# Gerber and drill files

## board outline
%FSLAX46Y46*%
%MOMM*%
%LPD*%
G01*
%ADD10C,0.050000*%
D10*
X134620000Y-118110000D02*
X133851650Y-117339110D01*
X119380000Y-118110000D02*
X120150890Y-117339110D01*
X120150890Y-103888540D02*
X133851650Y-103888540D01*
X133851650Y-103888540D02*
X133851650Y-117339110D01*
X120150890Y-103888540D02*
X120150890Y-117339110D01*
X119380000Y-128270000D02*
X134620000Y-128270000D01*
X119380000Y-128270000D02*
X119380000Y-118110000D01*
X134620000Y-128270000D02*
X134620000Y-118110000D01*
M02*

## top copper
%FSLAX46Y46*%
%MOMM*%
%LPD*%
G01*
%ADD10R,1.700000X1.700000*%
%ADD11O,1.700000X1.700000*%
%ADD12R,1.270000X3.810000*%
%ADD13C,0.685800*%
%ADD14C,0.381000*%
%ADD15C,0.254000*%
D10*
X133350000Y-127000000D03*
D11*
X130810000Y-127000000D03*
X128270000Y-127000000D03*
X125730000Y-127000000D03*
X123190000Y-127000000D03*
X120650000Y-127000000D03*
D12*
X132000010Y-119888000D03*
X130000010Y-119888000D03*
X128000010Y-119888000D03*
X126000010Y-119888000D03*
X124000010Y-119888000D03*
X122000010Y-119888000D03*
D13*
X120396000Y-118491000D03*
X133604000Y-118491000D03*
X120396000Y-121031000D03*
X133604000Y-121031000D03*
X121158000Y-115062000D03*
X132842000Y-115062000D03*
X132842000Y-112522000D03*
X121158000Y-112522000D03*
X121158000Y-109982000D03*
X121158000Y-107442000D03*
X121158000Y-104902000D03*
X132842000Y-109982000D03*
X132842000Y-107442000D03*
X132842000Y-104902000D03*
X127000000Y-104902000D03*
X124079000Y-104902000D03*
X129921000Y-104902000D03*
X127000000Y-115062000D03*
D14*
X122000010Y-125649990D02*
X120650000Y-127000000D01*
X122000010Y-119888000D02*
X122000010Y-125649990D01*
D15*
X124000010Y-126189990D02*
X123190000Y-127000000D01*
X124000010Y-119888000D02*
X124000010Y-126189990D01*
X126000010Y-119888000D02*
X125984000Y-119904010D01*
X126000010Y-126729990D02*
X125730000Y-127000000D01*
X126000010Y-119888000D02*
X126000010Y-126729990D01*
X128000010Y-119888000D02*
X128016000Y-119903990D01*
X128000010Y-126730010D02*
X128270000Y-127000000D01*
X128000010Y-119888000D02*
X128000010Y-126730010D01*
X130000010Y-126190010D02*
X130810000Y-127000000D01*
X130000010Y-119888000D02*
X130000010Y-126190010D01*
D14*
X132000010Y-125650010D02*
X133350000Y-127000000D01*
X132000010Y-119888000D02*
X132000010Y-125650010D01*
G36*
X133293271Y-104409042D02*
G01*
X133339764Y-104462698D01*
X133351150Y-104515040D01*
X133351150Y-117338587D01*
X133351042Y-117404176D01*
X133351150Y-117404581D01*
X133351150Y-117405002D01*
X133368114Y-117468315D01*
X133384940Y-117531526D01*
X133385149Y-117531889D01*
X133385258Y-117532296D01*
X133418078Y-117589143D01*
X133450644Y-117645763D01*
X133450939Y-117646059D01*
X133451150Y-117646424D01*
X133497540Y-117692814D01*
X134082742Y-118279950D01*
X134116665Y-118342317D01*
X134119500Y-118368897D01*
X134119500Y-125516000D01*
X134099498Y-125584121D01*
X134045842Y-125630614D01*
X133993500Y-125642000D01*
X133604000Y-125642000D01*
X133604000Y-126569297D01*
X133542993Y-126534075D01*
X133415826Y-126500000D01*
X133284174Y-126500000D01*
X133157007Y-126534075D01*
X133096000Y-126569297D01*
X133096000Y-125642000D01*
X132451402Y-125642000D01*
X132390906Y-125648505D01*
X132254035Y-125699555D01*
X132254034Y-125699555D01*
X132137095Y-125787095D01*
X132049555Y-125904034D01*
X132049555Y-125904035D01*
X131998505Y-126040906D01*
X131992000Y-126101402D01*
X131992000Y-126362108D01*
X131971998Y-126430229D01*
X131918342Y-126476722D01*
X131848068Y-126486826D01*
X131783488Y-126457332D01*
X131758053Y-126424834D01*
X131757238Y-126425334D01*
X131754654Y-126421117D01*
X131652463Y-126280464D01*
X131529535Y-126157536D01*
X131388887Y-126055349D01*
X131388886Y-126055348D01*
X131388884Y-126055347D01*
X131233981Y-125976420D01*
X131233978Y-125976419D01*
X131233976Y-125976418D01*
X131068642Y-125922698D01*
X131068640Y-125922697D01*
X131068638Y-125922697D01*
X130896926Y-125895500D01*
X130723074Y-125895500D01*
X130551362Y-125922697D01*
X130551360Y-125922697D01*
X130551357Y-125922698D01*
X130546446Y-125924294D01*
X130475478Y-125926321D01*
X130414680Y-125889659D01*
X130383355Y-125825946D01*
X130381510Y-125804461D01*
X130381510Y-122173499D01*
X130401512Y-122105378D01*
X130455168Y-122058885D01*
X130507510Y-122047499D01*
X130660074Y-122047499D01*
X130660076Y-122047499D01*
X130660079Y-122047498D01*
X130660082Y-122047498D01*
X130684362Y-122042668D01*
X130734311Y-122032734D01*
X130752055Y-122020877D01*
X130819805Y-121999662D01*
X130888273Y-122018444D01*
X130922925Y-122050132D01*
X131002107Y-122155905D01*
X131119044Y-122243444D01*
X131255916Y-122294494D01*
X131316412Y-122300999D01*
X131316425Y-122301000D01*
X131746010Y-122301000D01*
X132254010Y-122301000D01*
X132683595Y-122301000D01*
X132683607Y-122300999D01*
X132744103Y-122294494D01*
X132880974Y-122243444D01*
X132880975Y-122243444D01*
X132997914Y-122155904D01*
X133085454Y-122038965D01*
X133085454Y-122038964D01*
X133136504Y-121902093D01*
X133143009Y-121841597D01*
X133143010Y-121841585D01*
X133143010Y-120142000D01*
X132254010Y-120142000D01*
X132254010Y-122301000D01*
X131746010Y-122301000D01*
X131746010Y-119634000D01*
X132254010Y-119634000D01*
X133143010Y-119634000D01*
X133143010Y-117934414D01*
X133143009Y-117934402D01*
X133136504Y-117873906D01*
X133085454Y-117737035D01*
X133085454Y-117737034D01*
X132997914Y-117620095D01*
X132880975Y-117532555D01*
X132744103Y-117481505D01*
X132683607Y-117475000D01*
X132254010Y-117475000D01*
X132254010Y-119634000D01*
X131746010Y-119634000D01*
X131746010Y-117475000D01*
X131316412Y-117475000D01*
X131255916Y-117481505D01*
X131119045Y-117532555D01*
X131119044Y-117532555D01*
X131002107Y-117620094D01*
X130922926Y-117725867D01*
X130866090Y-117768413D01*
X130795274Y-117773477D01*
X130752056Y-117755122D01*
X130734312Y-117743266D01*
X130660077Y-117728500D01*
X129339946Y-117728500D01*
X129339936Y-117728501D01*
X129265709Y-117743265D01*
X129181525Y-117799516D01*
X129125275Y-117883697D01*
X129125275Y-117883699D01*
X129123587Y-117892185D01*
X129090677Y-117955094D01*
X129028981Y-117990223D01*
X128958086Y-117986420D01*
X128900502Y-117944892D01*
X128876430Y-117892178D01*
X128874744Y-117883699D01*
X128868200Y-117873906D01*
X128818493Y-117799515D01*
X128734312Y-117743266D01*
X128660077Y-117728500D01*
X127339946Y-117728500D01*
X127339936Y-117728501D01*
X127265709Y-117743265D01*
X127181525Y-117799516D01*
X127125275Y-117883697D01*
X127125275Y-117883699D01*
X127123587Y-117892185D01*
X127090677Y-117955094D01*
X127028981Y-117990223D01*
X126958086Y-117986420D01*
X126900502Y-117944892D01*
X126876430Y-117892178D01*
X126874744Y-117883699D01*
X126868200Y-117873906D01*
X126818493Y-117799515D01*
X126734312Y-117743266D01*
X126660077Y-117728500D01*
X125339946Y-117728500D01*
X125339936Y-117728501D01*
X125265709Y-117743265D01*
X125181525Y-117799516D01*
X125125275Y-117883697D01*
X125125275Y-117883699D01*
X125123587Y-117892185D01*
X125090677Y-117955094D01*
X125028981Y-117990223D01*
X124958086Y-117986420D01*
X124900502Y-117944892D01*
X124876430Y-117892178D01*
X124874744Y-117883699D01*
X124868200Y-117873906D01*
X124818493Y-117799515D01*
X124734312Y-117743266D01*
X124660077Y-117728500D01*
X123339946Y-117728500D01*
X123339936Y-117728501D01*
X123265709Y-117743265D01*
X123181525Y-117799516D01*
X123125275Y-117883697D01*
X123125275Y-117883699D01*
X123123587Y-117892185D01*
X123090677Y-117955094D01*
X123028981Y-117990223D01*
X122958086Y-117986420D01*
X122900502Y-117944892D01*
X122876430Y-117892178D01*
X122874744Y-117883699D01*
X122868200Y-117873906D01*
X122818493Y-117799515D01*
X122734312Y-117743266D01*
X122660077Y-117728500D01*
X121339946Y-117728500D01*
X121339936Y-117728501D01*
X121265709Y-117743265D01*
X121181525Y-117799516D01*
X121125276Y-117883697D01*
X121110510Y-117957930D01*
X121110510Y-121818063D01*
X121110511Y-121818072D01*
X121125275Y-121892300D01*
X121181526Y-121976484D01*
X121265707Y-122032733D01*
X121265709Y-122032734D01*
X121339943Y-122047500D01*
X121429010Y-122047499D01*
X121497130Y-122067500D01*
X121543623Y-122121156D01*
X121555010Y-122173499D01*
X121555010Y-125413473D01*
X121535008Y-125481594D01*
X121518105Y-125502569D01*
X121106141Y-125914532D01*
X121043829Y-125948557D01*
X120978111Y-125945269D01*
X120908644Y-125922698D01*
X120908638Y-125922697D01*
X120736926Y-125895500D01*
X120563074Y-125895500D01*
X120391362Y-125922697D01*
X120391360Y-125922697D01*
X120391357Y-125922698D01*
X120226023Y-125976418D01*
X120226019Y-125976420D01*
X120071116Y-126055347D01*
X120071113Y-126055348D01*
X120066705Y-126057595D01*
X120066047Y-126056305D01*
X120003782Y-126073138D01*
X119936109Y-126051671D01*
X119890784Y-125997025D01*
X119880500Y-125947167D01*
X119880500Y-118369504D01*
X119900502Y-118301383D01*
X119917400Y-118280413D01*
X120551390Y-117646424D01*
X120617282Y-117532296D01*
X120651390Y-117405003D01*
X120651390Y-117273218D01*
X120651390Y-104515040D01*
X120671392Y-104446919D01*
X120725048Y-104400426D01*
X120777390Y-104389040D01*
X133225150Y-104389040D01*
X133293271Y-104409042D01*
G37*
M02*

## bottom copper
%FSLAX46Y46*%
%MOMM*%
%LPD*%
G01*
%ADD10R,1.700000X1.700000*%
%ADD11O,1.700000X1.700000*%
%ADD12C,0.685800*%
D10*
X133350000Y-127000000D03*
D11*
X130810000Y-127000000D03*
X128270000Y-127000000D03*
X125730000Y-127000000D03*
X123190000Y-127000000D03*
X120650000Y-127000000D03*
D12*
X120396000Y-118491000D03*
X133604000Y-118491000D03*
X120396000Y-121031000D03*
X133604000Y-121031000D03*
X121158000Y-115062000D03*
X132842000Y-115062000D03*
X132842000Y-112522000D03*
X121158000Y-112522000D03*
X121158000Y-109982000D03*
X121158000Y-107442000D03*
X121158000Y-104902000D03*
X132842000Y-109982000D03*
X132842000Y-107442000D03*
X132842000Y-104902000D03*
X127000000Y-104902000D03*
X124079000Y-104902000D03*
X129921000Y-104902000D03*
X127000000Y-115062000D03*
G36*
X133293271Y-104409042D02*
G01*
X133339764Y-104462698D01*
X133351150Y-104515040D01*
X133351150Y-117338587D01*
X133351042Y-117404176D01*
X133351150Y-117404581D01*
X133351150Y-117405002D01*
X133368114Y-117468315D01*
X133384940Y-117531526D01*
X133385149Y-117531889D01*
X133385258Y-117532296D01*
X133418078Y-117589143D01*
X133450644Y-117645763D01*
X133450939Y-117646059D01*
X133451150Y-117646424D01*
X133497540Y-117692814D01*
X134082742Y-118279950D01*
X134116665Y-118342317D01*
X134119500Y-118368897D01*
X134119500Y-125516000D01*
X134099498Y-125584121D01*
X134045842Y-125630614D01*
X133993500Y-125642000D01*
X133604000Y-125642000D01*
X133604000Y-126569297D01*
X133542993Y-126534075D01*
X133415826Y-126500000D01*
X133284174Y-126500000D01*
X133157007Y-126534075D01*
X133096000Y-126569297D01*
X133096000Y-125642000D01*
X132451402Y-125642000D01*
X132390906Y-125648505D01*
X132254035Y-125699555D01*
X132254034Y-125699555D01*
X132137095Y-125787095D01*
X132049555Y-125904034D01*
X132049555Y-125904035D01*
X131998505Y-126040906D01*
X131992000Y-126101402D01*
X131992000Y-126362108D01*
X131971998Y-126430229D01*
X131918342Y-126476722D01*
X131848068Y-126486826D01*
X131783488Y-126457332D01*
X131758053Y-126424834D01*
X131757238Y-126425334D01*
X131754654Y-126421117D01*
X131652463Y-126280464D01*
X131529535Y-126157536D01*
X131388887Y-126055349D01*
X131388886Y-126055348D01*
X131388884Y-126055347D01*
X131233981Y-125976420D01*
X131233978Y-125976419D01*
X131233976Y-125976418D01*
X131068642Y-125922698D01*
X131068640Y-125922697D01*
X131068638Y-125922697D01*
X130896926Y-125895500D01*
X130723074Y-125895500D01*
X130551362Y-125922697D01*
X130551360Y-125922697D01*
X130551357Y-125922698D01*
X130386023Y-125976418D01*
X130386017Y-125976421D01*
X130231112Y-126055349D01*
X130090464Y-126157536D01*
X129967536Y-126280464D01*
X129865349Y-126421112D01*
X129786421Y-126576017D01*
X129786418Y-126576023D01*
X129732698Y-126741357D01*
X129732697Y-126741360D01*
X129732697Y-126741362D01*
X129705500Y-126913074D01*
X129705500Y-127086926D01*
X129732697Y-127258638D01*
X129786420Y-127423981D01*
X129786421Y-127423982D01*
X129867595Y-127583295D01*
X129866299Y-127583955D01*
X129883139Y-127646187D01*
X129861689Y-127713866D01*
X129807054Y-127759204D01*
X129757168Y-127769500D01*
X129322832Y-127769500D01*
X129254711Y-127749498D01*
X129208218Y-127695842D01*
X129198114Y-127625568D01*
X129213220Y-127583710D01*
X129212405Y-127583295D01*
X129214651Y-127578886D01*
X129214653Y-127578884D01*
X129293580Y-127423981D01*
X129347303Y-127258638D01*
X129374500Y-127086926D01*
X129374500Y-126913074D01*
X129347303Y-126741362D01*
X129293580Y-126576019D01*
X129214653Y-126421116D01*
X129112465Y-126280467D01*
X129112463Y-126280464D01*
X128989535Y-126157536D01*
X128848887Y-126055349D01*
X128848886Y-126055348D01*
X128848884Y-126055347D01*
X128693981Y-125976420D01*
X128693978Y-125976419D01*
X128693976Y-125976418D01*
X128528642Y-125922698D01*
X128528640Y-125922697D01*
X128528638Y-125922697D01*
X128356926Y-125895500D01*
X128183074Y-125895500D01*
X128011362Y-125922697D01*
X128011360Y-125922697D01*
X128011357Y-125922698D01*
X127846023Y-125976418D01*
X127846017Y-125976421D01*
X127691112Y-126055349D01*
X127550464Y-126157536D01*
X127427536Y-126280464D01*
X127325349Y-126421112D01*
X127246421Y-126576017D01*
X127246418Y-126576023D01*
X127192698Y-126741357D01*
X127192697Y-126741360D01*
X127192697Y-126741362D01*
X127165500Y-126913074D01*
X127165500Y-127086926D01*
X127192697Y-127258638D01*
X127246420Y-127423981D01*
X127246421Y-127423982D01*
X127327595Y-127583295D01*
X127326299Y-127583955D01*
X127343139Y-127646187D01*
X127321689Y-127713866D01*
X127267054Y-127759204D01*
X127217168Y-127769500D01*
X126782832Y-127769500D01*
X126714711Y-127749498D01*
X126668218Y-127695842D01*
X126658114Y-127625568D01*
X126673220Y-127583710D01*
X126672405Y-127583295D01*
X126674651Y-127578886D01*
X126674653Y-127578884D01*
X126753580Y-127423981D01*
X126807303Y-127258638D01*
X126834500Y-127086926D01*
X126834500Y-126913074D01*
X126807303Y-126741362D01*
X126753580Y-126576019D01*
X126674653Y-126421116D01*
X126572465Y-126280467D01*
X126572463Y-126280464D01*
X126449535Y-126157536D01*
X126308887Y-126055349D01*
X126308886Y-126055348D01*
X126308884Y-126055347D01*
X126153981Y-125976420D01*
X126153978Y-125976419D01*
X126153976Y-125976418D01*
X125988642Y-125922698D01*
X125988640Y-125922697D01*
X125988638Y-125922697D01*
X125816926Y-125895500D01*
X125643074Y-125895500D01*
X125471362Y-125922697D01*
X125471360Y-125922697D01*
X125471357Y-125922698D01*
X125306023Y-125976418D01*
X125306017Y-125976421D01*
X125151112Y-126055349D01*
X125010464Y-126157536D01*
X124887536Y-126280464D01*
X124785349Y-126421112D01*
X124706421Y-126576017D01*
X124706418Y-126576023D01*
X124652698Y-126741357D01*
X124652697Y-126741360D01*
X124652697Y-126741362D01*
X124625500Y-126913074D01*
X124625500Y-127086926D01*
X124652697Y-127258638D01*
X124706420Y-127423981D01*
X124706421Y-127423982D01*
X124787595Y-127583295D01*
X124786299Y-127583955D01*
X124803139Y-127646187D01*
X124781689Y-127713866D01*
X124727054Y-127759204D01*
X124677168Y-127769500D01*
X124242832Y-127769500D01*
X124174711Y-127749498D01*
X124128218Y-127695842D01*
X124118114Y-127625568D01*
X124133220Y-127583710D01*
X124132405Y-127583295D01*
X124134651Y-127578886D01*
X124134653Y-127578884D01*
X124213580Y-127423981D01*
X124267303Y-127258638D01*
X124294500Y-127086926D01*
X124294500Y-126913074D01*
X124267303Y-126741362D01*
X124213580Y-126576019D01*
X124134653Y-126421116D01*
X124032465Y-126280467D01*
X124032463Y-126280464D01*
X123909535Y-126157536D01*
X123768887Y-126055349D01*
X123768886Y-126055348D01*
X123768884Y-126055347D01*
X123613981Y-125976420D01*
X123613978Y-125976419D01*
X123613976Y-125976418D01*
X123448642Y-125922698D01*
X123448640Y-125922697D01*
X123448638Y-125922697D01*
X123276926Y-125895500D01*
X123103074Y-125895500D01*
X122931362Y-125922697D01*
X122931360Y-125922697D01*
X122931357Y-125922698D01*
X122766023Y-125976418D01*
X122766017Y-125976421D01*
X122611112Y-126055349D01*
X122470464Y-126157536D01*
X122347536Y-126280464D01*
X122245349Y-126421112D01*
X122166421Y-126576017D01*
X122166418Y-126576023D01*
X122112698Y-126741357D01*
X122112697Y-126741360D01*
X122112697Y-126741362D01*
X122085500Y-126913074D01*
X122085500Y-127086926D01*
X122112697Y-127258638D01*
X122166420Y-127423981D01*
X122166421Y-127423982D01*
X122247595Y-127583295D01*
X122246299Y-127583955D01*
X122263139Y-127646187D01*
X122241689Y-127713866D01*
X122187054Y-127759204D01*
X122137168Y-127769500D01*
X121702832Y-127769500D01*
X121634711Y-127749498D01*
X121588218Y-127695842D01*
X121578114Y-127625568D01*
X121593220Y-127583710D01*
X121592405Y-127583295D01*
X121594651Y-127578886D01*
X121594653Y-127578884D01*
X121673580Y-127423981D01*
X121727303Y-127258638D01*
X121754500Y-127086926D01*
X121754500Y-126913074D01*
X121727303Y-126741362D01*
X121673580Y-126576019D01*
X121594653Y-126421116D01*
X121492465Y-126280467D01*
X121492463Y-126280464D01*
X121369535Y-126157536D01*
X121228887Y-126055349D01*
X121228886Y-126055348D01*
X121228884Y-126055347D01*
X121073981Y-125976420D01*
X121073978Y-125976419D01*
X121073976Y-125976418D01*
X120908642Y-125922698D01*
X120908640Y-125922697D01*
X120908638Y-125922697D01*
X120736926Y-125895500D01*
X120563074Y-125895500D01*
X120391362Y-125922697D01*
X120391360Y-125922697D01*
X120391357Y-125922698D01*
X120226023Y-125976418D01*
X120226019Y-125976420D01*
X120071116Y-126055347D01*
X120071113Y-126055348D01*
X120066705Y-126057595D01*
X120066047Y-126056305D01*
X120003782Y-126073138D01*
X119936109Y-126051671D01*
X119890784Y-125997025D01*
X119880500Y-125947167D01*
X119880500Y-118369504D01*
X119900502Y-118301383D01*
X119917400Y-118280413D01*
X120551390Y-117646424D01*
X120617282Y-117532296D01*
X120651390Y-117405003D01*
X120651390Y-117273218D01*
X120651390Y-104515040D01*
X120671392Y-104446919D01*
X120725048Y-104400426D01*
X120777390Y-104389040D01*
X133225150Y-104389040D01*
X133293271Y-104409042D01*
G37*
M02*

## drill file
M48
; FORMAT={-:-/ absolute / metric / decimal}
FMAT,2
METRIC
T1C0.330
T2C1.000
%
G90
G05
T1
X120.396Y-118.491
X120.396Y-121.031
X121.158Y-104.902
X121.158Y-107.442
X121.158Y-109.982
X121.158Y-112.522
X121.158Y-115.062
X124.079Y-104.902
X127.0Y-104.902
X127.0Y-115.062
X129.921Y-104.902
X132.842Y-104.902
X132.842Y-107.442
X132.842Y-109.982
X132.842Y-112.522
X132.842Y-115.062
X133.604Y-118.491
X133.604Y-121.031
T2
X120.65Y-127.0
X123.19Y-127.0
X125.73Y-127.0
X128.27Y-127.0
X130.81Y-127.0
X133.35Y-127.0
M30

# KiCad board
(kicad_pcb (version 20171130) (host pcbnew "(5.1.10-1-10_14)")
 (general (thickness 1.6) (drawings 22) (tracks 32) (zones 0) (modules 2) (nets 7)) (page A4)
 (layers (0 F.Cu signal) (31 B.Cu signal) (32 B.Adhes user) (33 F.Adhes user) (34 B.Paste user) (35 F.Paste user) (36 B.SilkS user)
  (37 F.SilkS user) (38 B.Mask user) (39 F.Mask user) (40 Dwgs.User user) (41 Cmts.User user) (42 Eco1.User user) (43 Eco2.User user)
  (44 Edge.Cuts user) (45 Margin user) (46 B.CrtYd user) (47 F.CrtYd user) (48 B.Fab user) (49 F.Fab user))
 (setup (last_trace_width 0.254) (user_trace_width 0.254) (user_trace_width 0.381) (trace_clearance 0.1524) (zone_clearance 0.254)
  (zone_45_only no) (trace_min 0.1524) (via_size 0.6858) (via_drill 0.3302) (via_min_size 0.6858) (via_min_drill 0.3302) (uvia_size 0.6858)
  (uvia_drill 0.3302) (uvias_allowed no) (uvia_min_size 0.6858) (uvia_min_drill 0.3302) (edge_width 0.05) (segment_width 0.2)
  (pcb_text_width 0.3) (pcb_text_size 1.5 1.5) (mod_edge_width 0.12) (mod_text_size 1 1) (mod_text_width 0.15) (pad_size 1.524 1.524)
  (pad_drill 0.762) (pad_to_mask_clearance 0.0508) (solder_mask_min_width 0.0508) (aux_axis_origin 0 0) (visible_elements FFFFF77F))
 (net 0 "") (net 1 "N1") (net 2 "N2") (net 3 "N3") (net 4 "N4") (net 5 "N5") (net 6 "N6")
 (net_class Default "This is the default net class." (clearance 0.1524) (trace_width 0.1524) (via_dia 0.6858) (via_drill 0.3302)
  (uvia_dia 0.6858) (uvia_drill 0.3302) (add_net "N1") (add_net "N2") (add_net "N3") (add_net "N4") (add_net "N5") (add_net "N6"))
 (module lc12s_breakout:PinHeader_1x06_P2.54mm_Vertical (layer F.Cu) (at 133.35 127 270)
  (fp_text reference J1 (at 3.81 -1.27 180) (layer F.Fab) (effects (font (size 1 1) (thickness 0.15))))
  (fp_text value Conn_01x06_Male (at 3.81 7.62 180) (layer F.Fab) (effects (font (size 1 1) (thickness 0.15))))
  (pad 1 thru_hole rect (at 0 0 270) (size 1.7 1.7) (drill 1) (layers *.Cu *.Mask) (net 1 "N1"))
  (pad 2 thru_hole oval (at 0 2.54 270) (size 1.7 1.7) (drill 1) (layers *.Cu *.Mask) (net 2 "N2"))
  (pad 3 thru_hole oval (at 0 5.08 270) (size 1.7 1.7) (drill 1) (layers *.Cu *.Mask) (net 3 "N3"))
  (pad 4 thru_hole oval (at 0 7.62 270) (size 1.7 1.7) (drill 1) (layers *.Cu *.Mask) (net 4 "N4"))
  (pad 5 thru_hole oval (at 0 10.16 270) (size 1.7 1.7) (drill 1) (layers *.Cu *.Mask) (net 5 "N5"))
  (pad 6 thru_hole oval (at 0 12.7 270) (size 1.7 1.7) (drill 1) (layers *.Cu *.Mask) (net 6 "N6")))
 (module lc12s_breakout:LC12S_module (layer F.Cu) (at 122.00001 119.888)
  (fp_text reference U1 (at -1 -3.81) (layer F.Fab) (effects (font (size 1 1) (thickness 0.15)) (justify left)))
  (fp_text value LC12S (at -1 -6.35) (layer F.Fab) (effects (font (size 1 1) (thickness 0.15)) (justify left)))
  (pad 6 smd rect (at 10 0) (size 1.27 3.81) (layers F.Cu F.Paste F.Mask) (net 1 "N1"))
  (pad 5 smd rect (at 8 0) (size 1.27 3.81) (layers F.Cu F.Paste F.Mask) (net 2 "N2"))
  (pad 4 smd rect (at 6 0) (size 1.27 3.81) (layers F.Cu F.Paste F.Mask) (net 3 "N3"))
  (pad 3 smd rect (at 4 0) (size 1.27 3.81) (layers F.Cu F.Paste F.Mask) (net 4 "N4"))
  (pad 2 smd rect (at 2 0) (size 1.27 3.81) (layers F.Cu F.Paste F.Mask) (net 5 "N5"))
  (pad 1 smd rect (at 0 0) (size 1.27 3.81) (layers F.Cu F.Paste F.Mask) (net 6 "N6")))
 (gr_line (start 134.62 118.11) (end 133.85165 117.33911) (layer Edge.Cuts) (width 0.05))
 (gr_line (start 119.38 118.11) (end 120.15089 117.33911) (layer Edge.Cuts) (width 0.05))
 (gr_line (start 120.15089 103.88854) (end 133.85165 103.88854) (layer Edge.Cuts) (width 0.05))
 (gr_line (start 133.85165 103.88854) (end 133.85165 117.33911) (layer Edge.Cuts) (width 0.05))
 (gr_line (start 120.15089 103.88854) (end 120.15089 117.33911) (layer Edge.Cuts) (width 0.05))
 (gr_line (start 119.38 128.27) (end 134.62 128.27) (layer Edge.Cuts) (width 0.05))
 (gr_line (start 119.38 128.27) (end 119.38 118.11) (layer Edge.Cuts) (width 0.05))
 (gr_line (start 134.62 128.27) (end 134.62 118.11) (layer Edge.Cuts) (width 0.05))
 (segment (start 122.00001 125.64999) (end 120.65 127) (width 0.381) (layer F.Cu) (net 6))
 (segment (start 122.00001 119.888) (end 122.00001 125.64999) (width 0.381) (layer F.Cu) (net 6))
 (segment (start 124.00001 126.18999) (end 123.19 127) (width 0.254) (layer F.Cu) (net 5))
 (segment (start 124.00001 119.888) (end 124.00001 126.18999) (width 0.254) (layer F.Cu) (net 5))
 (segment (start 126.00001 119.888) (end 125.984 119.90401) (width 0.254) (layer F.Cu) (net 4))
 (segment (start 126.00001 126.72999) (end 125.73 127) (width 0.254) (layer F.Cu) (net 4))
 (segment (start 126.00001 119.888) (end 126.00001 126.72999) (width 0.254) (layer F.Cu) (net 4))
 (segment (start 128.00001 119.888) (end 128.016 119.90399) (width 0.254) (layer F.Cu) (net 3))
 (segment (start 128.00001 126.73001) (end 128.27 127) (width 0.254) (layer F.Cu) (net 3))
 (segment (start 128.00001 119.888) (end 128.00001 126.73001) (width 0.254) (layer F.Cu) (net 3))
 (segment (start 130.00001 126.19001) (end 130.81 127) (width 0.254) (layer F.Cu) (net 2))
 (segment (start 130.00001 119.888) (end 130.00001 126.19001) (width 0.254) (layer F.Cu) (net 2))
 (via (at 120.396 118.491) (size 0.6858) (drill 0.3302) (layers F.Cu B.Cu) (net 1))
 (via (at 133.604 118.491) (size 0.6858) (drill 0.3302) (layers F.Cu B.Cu) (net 1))
 (via (at 120.396 121.031) (size 0.6858) (drill 0.3302) (layers F.Cu B.Cu) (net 1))
 (via (at 133.604 121.031) (size 0.6858) (drill 0.3302) (layers F.Cu B.Cu) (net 1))
 (via (at 121.158 115.062) (size 0.6858) (drill 0.3302) (layers F.Cu B.Cu) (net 1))
 (via (at 132.842 115.062) (size 0.6858) (drill 0.3302) (layers F.Cu B.Cu) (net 1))
 (via (at 132.842 112.522) (size 0.6858) (drill 0.3302) (layers F.Cu B.Cu) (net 1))
 (via (at 121.158 112.522) (size 0.6858) (drill 0.3302) (layers F.Cu B.Cu) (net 1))
 (via (at 121.158 109.982) (size 0.6858) (drill 0.3302) (layers F.Cu B.Cu) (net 1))
 (via (at 121.158 107.442) (size 0.6858) (drill 0.3302) (layers F.Cu B.Cu) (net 1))
 (via (at 121.158 104.902) (size 0.6858) (drill 0.3302) (layers F.Cu B.Cu) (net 1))
 (via (at 132.842 109.982) (size 0.6858) (drill 0.3302) (layers F.Cu B.Cu) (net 1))
 (via (at 132.842 107.442) (size 0.6858) (drill 0.3302) (layers F.Cu B.Cu) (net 1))
 (via (at 132.842 104.902) (size 0.6858) (drill 0.3302) (layers F.Cu B.Cu) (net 1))
 (via (at 127 104.902) (size 0.6858) (drill 0.3302) (layers F.Cu B.Cu) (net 1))
 (via (at 124.079 104.902) (size 0.6858) (drill 0.3302) (layers F.Cu B.Cu) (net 1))
 (via (at 129.921 104.902) (size 0.6858) (drill 0.3302) (layers F.Cu B.Cu) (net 1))
 (via (at 127 115.062) (size 0.6858) (drill 0.3302) (layers F.Cu B.Cu) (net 1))
 (segment (start 132.00001 125.65001) (end 133.35 127) (width 0.381) (layer F.Cu) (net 1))
 (segment (start 132.00001 119.888) (end 132.00001 125.65001) (width 0.381) (layer F.Cu) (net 1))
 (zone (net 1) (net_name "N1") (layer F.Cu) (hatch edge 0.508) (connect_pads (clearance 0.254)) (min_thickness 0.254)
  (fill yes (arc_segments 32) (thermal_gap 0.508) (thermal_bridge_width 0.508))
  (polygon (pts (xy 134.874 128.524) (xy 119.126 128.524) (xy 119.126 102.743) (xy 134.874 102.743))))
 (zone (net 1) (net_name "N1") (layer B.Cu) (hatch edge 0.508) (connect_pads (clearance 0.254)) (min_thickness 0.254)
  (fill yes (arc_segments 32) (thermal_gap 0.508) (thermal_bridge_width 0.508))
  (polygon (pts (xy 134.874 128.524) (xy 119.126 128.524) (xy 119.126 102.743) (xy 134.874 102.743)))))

